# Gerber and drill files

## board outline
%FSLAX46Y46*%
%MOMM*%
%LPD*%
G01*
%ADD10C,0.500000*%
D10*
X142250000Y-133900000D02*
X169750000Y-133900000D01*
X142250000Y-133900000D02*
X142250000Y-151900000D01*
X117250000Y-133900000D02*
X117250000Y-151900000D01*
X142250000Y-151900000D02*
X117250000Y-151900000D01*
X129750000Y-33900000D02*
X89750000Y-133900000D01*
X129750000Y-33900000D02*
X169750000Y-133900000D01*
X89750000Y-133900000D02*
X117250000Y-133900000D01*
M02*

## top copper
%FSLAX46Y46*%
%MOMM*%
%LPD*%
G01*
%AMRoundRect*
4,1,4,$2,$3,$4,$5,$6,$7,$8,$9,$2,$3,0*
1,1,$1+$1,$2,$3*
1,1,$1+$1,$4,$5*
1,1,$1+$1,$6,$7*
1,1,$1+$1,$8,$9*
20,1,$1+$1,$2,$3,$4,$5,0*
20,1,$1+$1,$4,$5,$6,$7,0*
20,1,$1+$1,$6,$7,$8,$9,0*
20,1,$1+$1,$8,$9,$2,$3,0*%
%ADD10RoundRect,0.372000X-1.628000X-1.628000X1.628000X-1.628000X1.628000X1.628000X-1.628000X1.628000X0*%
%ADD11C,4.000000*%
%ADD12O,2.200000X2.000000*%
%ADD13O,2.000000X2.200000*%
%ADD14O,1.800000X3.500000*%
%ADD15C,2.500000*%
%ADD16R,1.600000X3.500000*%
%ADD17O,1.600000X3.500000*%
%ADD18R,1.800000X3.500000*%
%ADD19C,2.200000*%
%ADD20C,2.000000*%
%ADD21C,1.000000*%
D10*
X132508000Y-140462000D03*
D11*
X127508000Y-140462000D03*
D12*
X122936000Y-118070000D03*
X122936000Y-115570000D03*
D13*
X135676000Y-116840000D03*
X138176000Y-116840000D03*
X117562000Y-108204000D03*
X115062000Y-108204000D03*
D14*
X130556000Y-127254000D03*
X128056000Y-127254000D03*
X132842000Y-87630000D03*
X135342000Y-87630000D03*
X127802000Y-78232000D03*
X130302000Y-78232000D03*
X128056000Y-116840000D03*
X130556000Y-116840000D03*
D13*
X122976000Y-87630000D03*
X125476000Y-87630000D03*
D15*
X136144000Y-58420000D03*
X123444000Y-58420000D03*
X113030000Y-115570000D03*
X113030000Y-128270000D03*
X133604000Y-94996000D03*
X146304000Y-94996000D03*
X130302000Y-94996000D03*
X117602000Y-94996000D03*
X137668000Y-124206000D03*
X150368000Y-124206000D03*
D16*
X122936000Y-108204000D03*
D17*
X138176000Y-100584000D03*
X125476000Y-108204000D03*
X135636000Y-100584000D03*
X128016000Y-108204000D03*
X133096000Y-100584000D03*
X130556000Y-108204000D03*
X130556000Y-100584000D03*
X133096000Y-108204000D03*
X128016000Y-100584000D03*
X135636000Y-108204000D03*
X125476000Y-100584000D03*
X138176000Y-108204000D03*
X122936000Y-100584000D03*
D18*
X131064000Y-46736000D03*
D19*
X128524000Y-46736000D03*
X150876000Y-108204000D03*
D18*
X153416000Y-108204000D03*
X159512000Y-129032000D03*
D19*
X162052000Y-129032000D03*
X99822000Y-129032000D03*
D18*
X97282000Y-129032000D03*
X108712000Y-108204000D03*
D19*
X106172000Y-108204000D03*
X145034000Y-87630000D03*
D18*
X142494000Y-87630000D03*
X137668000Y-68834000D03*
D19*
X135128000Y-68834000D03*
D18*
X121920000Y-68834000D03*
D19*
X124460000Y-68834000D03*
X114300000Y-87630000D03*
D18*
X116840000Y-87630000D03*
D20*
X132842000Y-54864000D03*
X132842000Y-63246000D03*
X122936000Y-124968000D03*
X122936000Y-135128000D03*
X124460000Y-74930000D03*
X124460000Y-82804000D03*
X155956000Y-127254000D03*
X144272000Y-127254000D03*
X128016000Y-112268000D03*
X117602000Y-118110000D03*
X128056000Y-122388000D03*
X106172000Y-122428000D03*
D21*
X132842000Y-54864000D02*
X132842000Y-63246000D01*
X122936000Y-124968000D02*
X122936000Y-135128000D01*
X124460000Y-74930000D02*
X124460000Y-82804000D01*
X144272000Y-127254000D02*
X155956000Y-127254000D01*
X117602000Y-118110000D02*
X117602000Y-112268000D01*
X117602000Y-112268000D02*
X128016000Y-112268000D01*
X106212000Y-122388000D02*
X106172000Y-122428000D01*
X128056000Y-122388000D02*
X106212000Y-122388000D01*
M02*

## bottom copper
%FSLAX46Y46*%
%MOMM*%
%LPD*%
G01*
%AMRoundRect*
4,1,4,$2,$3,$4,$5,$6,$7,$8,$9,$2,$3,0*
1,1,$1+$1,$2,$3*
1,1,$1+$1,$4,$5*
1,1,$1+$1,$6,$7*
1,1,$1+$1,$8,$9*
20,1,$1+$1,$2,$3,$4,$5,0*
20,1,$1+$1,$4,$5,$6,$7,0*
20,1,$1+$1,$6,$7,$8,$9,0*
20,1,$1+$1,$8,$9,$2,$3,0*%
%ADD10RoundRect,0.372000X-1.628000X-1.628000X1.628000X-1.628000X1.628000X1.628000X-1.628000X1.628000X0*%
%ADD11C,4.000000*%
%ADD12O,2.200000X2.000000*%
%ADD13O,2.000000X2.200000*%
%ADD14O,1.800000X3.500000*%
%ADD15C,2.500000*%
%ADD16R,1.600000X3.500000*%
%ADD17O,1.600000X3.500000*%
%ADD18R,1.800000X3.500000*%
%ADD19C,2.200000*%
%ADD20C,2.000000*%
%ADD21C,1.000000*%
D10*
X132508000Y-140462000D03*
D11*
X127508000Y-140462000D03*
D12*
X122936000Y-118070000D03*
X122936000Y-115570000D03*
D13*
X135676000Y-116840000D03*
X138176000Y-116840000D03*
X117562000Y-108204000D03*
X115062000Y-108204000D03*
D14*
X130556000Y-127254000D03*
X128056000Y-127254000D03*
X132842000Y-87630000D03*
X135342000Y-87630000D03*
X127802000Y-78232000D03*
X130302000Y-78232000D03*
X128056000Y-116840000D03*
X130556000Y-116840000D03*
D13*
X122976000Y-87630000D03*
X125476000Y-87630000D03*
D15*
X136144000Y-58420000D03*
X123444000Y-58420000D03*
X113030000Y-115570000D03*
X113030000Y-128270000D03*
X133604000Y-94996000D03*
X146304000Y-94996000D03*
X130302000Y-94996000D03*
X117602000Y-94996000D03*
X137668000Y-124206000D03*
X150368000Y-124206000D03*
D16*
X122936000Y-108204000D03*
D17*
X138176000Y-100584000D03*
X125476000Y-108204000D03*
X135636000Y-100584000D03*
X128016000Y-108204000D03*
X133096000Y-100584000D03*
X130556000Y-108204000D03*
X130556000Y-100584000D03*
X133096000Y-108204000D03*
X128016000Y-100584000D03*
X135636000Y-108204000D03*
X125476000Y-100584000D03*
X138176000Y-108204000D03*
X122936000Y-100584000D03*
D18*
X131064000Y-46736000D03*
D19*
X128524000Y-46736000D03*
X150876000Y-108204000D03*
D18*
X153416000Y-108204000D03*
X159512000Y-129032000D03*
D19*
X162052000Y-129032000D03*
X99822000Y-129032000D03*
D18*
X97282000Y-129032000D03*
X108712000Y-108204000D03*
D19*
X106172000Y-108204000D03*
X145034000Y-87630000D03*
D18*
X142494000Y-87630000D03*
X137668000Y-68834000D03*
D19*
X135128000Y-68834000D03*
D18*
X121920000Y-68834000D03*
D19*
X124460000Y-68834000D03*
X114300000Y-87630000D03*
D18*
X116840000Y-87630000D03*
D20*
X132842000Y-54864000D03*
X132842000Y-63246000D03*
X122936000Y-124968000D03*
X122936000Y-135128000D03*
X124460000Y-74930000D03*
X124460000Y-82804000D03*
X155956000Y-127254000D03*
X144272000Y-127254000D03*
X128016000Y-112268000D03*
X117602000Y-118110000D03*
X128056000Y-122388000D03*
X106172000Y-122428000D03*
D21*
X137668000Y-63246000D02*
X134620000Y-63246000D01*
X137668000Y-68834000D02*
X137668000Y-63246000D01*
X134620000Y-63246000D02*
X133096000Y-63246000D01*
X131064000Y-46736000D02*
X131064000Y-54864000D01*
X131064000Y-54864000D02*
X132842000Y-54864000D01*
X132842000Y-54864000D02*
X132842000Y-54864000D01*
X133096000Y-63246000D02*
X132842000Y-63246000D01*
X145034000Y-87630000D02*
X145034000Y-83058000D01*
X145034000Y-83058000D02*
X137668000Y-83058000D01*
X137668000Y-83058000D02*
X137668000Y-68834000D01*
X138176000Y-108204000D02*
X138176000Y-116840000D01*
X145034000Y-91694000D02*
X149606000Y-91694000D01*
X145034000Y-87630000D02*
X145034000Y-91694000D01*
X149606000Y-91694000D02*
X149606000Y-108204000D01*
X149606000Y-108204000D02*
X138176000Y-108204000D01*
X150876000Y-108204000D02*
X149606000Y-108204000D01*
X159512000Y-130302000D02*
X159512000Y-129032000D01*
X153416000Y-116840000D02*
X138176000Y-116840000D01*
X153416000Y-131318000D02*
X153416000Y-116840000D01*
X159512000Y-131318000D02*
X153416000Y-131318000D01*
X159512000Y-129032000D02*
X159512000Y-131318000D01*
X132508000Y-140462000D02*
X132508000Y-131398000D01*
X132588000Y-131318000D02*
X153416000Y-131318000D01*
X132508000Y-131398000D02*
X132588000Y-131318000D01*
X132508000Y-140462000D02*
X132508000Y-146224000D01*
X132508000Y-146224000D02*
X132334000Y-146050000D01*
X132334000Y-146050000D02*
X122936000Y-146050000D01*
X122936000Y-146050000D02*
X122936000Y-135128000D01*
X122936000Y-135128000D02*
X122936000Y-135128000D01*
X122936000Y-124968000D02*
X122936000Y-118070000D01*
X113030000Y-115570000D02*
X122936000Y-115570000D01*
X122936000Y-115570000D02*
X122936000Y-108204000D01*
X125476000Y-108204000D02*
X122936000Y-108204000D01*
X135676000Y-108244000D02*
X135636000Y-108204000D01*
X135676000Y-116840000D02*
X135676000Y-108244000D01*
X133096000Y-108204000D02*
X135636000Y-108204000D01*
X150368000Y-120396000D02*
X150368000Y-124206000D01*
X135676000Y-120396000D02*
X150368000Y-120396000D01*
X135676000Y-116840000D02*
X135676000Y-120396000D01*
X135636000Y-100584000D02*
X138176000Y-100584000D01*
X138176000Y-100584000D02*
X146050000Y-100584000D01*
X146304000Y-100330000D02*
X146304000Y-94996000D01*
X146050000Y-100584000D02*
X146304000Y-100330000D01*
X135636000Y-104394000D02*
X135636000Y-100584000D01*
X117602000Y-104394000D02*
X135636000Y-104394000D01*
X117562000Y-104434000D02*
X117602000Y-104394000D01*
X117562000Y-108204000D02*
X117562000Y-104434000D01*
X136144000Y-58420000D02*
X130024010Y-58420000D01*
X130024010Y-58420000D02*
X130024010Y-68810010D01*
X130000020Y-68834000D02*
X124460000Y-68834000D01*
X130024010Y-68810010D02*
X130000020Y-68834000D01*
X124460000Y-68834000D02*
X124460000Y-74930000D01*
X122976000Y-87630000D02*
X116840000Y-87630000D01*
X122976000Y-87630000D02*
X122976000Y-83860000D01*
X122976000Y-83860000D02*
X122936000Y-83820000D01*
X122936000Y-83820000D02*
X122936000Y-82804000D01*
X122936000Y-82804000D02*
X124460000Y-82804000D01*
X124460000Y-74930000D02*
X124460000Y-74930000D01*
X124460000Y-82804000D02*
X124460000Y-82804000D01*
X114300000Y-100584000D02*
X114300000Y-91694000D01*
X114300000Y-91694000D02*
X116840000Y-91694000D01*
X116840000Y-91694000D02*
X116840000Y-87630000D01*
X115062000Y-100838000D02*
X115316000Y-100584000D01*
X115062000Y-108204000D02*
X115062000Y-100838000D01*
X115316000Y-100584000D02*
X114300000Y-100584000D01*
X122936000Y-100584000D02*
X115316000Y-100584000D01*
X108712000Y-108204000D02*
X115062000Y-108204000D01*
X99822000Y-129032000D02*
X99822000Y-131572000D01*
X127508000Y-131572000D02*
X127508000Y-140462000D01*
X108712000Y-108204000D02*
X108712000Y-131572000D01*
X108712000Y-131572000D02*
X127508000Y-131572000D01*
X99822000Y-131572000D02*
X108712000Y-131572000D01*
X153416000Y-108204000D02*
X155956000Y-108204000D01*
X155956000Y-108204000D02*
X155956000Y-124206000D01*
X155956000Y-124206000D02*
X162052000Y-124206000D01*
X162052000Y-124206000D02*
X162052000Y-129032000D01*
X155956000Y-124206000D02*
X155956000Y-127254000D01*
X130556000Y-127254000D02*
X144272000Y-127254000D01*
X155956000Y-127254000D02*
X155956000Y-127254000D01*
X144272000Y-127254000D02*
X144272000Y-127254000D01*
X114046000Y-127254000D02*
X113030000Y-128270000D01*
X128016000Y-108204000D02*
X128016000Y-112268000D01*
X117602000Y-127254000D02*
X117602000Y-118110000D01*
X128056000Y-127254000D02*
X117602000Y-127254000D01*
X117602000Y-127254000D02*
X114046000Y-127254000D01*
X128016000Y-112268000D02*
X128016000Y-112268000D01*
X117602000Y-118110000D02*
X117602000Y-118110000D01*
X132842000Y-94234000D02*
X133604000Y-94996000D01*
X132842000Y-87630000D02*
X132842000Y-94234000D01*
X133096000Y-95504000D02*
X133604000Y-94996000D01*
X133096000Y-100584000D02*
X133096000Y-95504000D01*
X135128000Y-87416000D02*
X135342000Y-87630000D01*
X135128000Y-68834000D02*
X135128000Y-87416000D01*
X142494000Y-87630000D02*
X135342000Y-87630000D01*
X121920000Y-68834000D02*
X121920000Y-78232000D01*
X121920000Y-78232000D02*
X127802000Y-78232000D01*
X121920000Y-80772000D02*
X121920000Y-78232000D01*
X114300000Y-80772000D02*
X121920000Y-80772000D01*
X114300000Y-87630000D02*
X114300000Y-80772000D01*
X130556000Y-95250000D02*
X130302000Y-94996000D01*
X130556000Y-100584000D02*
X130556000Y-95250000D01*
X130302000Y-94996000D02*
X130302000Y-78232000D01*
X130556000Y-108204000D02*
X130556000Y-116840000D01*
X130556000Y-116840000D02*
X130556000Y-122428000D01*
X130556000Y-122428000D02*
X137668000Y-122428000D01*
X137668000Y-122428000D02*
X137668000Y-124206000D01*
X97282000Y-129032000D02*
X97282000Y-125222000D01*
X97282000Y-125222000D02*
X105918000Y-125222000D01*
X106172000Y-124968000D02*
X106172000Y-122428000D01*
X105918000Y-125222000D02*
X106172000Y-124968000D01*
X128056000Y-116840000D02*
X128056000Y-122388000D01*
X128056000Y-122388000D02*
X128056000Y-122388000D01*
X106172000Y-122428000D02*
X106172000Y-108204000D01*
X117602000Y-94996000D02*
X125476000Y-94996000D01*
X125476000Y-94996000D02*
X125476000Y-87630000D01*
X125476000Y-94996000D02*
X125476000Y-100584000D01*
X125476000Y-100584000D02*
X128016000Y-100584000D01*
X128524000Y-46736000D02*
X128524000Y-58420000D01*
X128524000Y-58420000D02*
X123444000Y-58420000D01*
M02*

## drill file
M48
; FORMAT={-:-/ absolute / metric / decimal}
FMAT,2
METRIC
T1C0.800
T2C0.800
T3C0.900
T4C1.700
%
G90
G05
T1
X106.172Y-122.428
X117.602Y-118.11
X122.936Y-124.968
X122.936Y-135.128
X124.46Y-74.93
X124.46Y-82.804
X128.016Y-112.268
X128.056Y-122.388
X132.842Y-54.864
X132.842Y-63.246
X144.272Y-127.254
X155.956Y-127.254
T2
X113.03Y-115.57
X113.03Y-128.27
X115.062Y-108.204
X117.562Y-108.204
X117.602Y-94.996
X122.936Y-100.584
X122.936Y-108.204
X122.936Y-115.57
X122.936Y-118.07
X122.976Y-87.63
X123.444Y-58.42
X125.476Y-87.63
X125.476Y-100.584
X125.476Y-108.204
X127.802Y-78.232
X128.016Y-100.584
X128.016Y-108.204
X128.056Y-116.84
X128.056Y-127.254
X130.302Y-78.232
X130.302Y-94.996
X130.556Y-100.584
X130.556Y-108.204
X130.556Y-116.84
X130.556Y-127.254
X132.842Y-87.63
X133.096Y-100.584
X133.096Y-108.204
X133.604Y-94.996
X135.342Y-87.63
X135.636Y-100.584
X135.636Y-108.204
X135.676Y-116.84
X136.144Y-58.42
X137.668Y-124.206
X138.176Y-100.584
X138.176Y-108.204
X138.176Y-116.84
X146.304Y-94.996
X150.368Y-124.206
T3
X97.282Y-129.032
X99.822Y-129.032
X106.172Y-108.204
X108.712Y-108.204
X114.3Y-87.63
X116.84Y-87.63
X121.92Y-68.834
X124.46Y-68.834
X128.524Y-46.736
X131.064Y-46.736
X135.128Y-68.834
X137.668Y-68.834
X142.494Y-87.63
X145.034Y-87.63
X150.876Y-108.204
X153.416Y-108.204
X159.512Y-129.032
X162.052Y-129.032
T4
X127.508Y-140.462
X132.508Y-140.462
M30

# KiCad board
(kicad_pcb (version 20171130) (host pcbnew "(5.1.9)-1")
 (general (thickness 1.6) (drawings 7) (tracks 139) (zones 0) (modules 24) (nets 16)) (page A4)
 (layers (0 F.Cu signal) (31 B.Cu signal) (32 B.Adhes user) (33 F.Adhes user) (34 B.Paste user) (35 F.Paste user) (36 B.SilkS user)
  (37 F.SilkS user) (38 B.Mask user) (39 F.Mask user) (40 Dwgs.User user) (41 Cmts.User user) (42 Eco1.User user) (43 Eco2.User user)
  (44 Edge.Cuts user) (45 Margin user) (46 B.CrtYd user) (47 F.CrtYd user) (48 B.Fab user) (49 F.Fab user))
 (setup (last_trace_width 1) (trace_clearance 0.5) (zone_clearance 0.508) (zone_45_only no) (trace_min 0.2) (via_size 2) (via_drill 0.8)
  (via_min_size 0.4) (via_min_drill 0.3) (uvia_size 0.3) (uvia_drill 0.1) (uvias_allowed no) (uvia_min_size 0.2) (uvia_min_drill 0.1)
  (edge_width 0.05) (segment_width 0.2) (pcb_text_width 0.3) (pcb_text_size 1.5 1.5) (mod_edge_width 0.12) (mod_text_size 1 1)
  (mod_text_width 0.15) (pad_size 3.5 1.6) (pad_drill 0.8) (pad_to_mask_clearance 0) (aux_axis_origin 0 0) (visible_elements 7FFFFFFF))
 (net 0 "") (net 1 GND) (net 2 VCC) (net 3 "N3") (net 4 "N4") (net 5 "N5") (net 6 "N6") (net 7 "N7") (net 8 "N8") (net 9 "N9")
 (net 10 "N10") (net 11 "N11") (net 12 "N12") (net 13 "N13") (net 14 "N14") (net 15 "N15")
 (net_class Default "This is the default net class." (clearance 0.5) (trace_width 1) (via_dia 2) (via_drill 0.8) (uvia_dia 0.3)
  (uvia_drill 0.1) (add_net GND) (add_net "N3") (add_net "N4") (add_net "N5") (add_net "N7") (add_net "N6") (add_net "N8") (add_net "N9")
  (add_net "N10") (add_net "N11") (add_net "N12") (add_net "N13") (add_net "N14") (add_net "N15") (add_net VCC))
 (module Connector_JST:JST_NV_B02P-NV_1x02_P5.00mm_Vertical (layer F.Cu) (at 127.508 140.462)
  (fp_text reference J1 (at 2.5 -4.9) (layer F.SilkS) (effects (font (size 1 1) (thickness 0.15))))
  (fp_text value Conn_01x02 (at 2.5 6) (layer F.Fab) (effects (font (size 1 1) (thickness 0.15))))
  (pad 2 thru_hole roundrect (at 5 0) (size 4 4) (drill 1.7) (layers *.Cu *.Mask) (roundrect_rratio 0.09300000000000001) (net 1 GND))
  (pad 1 thru_hole circle (at 0 0) (size 4 4) (drill 1.7) (layers *.Cu *.Mask) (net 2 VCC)))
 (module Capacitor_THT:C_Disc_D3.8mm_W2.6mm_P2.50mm (layer F.Cu) (at 122.936 115.57 270)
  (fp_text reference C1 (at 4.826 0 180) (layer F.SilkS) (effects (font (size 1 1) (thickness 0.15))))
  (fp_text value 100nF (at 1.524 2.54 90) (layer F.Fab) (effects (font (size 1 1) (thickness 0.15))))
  (pad 2 thru_hole oval (at 2.5 0 270) (size 2 2.2) (drill 0.8) (layers *.Cu *.Mask) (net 1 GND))
  (pad 1 thru_hole oval (at 0 0 270) (size 2 2.2) (drill 0.8) (layers *.Cu *.Mask) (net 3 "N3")))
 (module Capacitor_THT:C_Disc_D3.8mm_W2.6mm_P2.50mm (layer F.Cu) (at 135.676 116.84)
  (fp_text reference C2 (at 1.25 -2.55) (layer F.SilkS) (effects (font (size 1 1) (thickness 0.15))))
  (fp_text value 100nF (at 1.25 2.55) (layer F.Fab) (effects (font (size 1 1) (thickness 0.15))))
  (pad 1 thru_hole oval (at 0 0) (size 2 2.2) (drill 0.8) (layers *.Cu *.Mask) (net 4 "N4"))
  (pad 2 thru_hole oval (at 2.5 0) (size 2 2.2) (drill 0.8) (layers *.Cu *.Mask) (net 1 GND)))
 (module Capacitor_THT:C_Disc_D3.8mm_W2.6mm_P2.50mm (layer F.Cu) (at 115.062 108.204)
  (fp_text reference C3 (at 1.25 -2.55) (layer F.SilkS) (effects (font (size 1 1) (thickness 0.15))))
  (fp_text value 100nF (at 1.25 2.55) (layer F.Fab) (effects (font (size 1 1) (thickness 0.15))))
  (pad 2 thru_hole oval (at 2.5 0) (size 2 2.2) (drill 0.8) (layers *.Cu *.Mask) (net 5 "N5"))
  (pad 1 thru_hole oval (at 0 0) (size 2 2.2) (drill 0.8) (layers *.Cu *.Mask) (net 2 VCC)))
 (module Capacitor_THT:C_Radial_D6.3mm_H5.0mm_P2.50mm (layer F.Cu) (at 128.056 127.254)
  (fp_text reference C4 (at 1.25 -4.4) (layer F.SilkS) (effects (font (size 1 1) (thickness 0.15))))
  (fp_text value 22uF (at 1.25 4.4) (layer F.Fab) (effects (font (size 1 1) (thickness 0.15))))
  (pad 2 thru_hole oval (at 2.5 0) (size 1.8 3.5) (drill 0.8) (layers *.Cu *.Mask) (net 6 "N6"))
  (pad 1 thru_hole oval (at 0 0) (size 1.8 3.5) (drill 0.8) (layers *.Cu *.Mask) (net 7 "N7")))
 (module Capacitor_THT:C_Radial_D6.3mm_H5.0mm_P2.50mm (layer F.Cu) (at 132.842 87.63)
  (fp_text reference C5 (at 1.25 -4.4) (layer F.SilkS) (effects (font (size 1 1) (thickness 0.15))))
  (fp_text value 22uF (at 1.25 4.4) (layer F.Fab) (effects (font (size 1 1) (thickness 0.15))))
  (pad 1 thru_hole oval (at 0 0) (size 1.8 3.5) (drill 0.8) (layers *.Cu *.Mask) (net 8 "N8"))
  (pad 2 thru_hole oval (at 2.5 0) (size 1.8 3.5) (drill 0.8) (layers *.Cu *.Mask) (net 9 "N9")))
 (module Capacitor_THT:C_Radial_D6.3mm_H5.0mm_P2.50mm (layer F.Cu) (at 127.802 78.232)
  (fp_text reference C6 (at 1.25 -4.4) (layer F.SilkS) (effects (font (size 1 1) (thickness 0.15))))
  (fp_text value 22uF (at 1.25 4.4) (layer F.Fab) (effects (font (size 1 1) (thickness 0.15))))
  (pad 1 thru_hole oval (at 0 0) (size 1.8 3.5) (drill 0.8) (layers *.Cu *.Mask) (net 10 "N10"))
  (pad 2 thru_hole oval (at 2.5 0) (size 1.8 3.5) (drill 0.8) (layers *.Cu *.Mask) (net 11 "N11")))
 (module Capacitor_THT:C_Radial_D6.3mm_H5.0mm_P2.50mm (layer F.Cu) (at 128.056 116.84)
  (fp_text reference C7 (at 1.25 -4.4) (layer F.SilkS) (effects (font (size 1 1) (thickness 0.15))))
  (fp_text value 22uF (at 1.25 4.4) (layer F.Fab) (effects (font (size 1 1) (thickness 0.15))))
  (pad 1 thru_hole oval (at 0 0) (size 1.8 3.5) (drill 0.8) (layers *.Cu *.Mask) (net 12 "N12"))
  (pad 2 thru_hole oval (at 2.5 0) (size 1.8 3.5) (drill 0.8) (layers *.Cu *.Mask) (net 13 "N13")))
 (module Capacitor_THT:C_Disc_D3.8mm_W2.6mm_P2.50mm (layer F.Cu) (at 122.976 87.63)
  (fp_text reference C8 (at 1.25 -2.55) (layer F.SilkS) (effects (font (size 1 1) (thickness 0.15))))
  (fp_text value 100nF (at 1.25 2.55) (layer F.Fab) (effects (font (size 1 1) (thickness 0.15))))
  (pad 1 thru_hole oval (at 0 0) (size 2 2.2) (drill 0.8) (layers *.Cu *.Mask) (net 2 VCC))
  (pad 2 thru_hole oval (at 2.5 0) (size 2 2.2) (drill 0.8) (layers *.Cu *.Mask) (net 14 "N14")))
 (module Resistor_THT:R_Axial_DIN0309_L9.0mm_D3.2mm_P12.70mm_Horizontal (layer F.Cu) (at 136.144 58.42 180)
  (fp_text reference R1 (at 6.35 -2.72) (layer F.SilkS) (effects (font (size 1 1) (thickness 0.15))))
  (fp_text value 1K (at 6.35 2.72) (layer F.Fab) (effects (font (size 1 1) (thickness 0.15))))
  (pad 1 thru_hole circle (at 0 0 180) (size 2.5 2.5) (drill 0.8) (layers *.Cu *.Mask) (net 2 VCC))
  (pad 2 thru_hole circle (at 12.7 0 180) (size 2.5 2.5) (drill 0.8) (layers *.Cu *.Mask) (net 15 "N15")))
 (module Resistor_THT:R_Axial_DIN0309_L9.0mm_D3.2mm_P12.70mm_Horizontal (layer F.Cu) (at 113.03 128.27 90)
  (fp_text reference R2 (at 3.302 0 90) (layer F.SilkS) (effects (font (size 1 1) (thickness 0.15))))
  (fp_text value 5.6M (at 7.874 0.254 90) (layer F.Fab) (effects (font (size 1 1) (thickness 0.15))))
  (pad 2 thru_hole circle (at 12.7 0 90) (size 2.5 2.5) (drill 0.8) (layers *.Cu *.Mask) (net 3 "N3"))
  (pad 1 thru_hole circle (at 0 0 90) (size 2.5 2.5) (drill 0.8) (layers *.Cu *.Mask) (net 7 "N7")))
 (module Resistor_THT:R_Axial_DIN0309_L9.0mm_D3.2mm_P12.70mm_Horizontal (layer F.Cu) (at 133.604 94.996)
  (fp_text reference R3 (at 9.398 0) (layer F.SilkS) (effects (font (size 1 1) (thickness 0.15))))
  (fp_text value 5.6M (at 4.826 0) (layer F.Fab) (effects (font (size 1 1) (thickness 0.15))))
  (pad 1 thru_hole circle (at 0 0) (size 2.5 2.5) (drill 0.8) (layers *.Cu *.Mask) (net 8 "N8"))
  (pad 2 thru_hole circle (at 12.7 0) (size 2.5 2.5) (drill 0.8) (layers *.Cu *.Mask) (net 5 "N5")))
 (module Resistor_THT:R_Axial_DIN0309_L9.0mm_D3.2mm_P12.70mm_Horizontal (layer F.Cu) (at 130.302 94.996 180)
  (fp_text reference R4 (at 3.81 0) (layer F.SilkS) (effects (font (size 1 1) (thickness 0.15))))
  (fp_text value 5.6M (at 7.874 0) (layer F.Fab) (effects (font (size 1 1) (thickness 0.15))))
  (pad 1 thru_hole circle (at 0 0 180) (size 2.5 2.5) (drill 0.8) (layers *.Cu *.Mask) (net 11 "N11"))
  (pad 2 thru_hole circle (at 12.7 0 180) (size 2.5 2.5) (drill 0.8) (layers *.Cu *.Mask) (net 14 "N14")))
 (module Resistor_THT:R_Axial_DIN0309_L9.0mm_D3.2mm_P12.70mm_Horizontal (layer F.Cu) (at 137.668 124.206)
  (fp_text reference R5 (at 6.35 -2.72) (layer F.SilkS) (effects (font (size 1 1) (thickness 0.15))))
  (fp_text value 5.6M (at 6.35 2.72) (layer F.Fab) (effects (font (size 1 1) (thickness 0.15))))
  (pad 1 thru_hole circle (at 0 0) (size 2.5 2.5) (drill 0.8) (layers *.Cu *.Mask) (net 13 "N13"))
  (pad 2 thru_hole circle (at 12.7 0) (size 2.5 2.5) (drill 0.8) (layers *.Cu *.Mask) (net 4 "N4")))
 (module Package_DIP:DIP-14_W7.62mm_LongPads (layer F.Cu) (at 122.936 108.204 90)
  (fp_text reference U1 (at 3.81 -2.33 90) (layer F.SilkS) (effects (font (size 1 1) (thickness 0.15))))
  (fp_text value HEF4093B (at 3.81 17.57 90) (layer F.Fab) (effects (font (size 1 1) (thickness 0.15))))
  (pad 1 thru_hole rect (at 0 0 90) (size 3.5 1.6) (drill 0.8) (layers *.Cu *.Mask) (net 3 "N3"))
  (pad 8 thru_hole oval (at 7.62 15.24 90) (size 3.5 1.6) (drill 0.8) (layers *.Cu *.Mask) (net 5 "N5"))
  (pad 2 thru_hole oval (at 0 2.54 90) (size 3.5 1.6) (drill 0.8) (layers *.Cu *.Mask) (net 3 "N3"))
  (pad 9 thru_hole oval (at 7.62 12.7 90) (size 3.5 1.6) (drill 0.8) (layers *.Cu *.Mask) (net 5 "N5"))
  (pad 3 thru_hole oval (at 0 5.08 90) (size 3.5 1.6) (drill 0.8) (layers *.Cu *.Mask) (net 7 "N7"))
  (pad 10 thru_hole oval (at 7.62 10.16 90) (size 3.5 1.6) (drill 0.8) (layers *.Cu *.Mask) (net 8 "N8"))
  (pad 4 thru_hole oval (at 0 7.62 90) (size 3.5 1.6) (drill 0.8) (layers *.Cu *.Mask) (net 13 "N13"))
  (pad 11 thru_hole oval (at 7.62 7.62 90) (size 3.5 1.6) (drill 0.8) (layers *.Cu *.Mask) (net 11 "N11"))
  (pad 5 thru_hole oval (at 0 10.16 90) (size 3.5 1.6) (drill 0.8) (layers *.Cu *.Mask) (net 4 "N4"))
  (pad 12 thru_hole oval (at 7.62 5.08 90) (size 3.5 1.6) (drill 0.8) (layers *.Cu *.Mask) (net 14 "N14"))
  (pad 6 thru_hole oval (at 0 12.7 90) (size 3.5 1.6) (drill 0.8) (layers *.Cu *.Mask) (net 4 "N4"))
  (pad 13 thru_hole oval (at 7.62 2.54 90) (size 3.5 1.6) (drill 0.8) (layers *.Cu *.Mask) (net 14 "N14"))
  (pad 7 thru_hole oval (at 0 15.24 90) (size 3.5 1.6) (drill 0.8) (layers *.Cu *.Mask) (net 1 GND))
  (pad 14 thru_hole oval (at 7.62 0 90) (size 3.5 1.6) (drill 0.8) (layers *.Cu *.Mask) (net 2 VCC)))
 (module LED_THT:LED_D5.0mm (layer F.Cu) (at 131.064 46.736 180)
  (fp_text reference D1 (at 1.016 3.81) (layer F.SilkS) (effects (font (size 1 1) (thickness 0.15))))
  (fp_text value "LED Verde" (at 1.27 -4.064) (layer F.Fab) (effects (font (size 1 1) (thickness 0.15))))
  (pad 1 thru_hole rect (at 0 0 180) (size 1.8 3.5) (drill 0.9) (layers *.Cu *.Mask) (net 1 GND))
  (pad 2 thru_hole circle (at 2.54 0 180) (size 2.2 2.2) (drill 0.9) (layers *.Cu *.Mask) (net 15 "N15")))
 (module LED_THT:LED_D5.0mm (layer F.Cu) (at 153.416 108.204 180)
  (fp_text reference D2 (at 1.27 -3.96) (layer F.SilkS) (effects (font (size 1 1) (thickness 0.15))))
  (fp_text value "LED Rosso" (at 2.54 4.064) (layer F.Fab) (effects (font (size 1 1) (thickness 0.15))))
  (pad 2 thru_hole circle (at 2.54 0 180) (size 2.2 2.2) (drill 0.9) (layers *.Cu *.Mask) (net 1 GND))
  (pad 1 thru_hole rect (at 0 0 180) (size 1.8 3.5) (drill 0.9) (layers *.Cu *.Mask) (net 6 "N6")))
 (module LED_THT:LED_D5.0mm (layer F.Cu) (at 159.512 129.032)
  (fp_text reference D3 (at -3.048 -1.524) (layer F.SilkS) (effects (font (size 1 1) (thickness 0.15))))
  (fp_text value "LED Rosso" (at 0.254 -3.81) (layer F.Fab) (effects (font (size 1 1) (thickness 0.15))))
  (pad 1 thru_hole rect (at 0 0) (size 1.8 3.5) (drill 0.9) (layers *.Cu *.Mask) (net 1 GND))
  (pad 2 thru_hole circle (at 2.54 0) (size 2.2 2.2) (drill 0.9) (layers *.Cu *.Mask) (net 6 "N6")))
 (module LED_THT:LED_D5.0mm (layer F.Cu) (at 97.282 129.032)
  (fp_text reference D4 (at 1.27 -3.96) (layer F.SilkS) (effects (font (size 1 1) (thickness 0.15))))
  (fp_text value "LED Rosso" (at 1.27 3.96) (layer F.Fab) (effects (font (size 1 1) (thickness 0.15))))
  (pad 2 thru_hole circle (at 2.54 0) (size 2.2 2.2) (drill 0.9) (layers *.Cu *.Mask) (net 2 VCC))
  (pad 1 thru_hole rect (at 0 0) (size 1.8 3.5) (drill 0.9) (layers *.Cu *.Mask) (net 12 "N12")))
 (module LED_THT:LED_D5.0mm (layer F.Cu) (at 108.712 108.204 180)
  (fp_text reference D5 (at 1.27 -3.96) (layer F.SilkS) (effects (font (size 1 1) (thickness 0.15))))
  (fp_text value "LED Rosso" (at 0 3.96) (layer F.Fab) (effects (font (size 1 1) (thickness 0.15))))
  (pad 1 thru_hole rect (at 0 0 180) (size 1.8 3.5) (drill 0.9) (layers *.Cu *.Mask) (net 2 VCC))
  (pad 2 thru_hole circle (at 2.54 0 180) (size 2.2 2.2) (drill 0.9) (layers *.Cu *.Mask) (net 12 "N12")))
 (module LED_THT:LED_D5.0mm (layer F.Cu) (at 142.494 87.63)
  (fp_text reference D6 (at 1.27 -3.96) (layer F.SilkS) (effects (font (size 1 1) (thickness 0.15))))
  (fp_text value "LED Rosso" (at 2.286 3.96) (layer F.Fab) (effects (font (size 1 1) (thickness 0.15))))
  (pad 2 thru_hole circle (at 2.54 0) (size 2.2 2.2) (drill 0.9) (layers *.Cu *.Mask) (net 1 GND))
  (pad 1 thru_hole rect (at 0 0) (size 1.8 3.5) (drill 0.9) (layers *.Cu *.Mask) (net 9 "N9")))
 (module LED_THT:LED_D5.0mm (layer F.Cu) (at 137.668 68.834 180)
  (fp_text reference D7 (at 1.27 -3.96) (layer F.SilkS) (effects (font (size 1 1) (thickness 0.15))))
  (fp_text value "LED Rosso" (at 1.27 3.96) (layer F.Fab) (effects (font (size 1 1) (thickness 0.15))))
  (pad 1 thru_hole rect (at 0 0 180) (size 1.8 3.5) (drill 0.9) (layers *.Cu *.Mask) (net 1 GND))
  (pad 2 thru_hole circle (at 2.54 0 180) (size 2.2 2.2) (drill 0.9) (layers *.Cu *.Mask) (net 9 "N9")))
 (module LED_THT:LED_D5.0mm (layer F.Cu) (at 121.92 68.834)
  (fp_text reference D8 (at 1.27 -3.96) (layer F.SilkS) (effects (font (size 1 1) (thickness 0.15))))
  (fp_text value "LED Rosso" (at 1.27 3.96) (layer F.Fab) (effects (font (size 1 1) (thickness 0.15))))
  (pad 1 thru_hole rect (at 0 0) (size 1.8 3.5) (drill 0.9) (layers *.Cu *.Mask) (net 10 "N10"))
  (pad 2 thru_hole circle (at 2.54 0) (size 2.2 2.2) (drill 0.9) (layers *.Cu *.Mask) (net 2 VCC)))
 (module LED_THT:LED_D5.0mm (layer F.Cu) (at 116.84 87.63 180)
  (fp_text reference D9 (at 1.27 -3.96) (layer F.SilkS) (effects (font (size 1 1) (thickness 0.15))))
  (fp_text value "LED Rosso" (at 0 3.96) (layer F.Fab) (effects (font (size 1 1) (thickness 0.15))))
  (pad 2 thru_hole circle (at 2.54 0 180) (size 2.2 2.2) (drill 0.9) (layers *.Cu *.Mask) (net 10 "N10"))
  (pad 1 thru_hole rect (at 0 0 180) (size 1.8 3.5) (drill 0.9) (layers *.Cu *.Mask) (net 2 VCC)))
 (gr_line (start 142.25 133.9) (end 169.75 133.9) (layer Edge.Cuts) (width 0.5))
 (gr_line (start 142.25 133.9) (end 142.25 151.9) (layer Edge.Cuts) (width 0.5))
 (gr_line (start 117.25 133.9) (end 117.25 151.9) (layer Edge.Cuts) (width 0.5))
 (gr_line (start 142.25 151.9) (end 117.25 151.9) (layer Edge.Cuts) (width 0.5))
 (gr_line (start 129.75 33.9) (end 89.75 133.9) (layer Edge.Cuts) (width 0.5))
 (gr_line (start 129.75 33.9) (end 169.75 133.9) (layer Edge.Cuts) (width 0.5))
 (gr_line (start 89.75 133.9) (end 117.25 133.9) (layer Edge.Cuts) (width 0.5))
 (segment (start 137.668 63.246) (end 134.62 63.246) (width 1) (layer B.Cu) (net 1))
 (segment (start 137.668 68.834) (end 137.668 63.246) (width 1) (layer B.Cu) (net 1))
 (segment (start 134.62 63.246) (end 133.096 63.246) (width 1) (layer B.Cu) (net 1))
 (segment (start 131.064 46.736) (end 131.064 54.864) (width 1) (layer B.Cu) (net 1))
 (segment (start 131.064 54.864) (end 132.842 54.864) (width 1) (layer B.Cu) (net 1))
 (segment (start 132.842 54.864) (end 132.842 54.864) (width 1) (layer B.Cu) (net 1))
 (via (at 132.842 54.864) (size 2) (drill 0.8) (layers F.Cu B.Cu) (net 1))
 (segment (start 133.096 63.246) (end 132.842 63.246) (width 1) (layer B.Cu) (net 1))
 (via (at 132.842 63.246) (size 2) (drill 0.8) (layers F.Cu B.Cu) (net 1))
 (segment (start 132.842 54.864) (end 132.842 63.246) (width 1) (layer F.Cu) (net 1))
 (segment (start 145.034 87.63) (end 145.034 83.058) (width 1) (layer B.Cu) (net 1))
 (segment (start 145.034 83.058) (end 137.668 83.058) (width 1) (layer B.Cu) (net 1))
 (segment (start 137.668 83.058) (end 137.668 68.834) (width 1) (layer B.Cu) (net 1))
 (segment (start 138.176 108.204) (end 138.176 116.84) (width 1) (layer B.Cu) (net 1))
 (segment (start 145.034 91.694) (end 149.606 91.694) (width 1) (layer B.Cu) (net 1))
 (segment (start 145.034 87.63) (end 145.034 91.694) (width 1) (layer B.Cu) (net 1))
 (segment (start 149.606 91.694) (end 149.606 108.204) (width 1) (layer B.Cu) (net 1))
 (segment (start 149.606 108.204) (end 138.176 108.204) (width 1) (layer B.Cu) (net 1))
 (segment (start 150.876 108.204) (end 149.606 108.204) (width 1) (layer B.Cu) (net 1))
 (segment (start 159.512 130.302) (end 159.512 129.032) (width 1) (layer B.Cu) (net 1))
 (segment (start 153.416 116.84) (end 138.176 116.84) (width 1) (layer B.Cu) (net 1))
 (segment (start 153.416 131.318) (end 153.416 116.84) (width 1) (layer B.Cu) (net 1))
 (segment (start 159.512 131.318) (end 153.416 131.318) (width 1) (layer B.Cu) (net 1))
 (segment (start 159.512 129.032) (end 159.512 131.318) (width 1) (layer B.Cu) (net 1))
 (segment (start 132.508 140.462) (end 132.508 131.398) (width 1) (layer B.Cu) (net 1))
 (segment (start 132.588 131.318) (end 153.416 131.318) (width 1) (layer B.Cu) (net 1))
 (segment (start 132.508 131.398) (end 132.588 131.318) (width 1) (layer B.Cu) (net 1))
 (segment (start 132.508 140.462) (end 132.508 146.224) (width 1) (layer B.Cu) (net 1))
 (segment (start 132.508 146.224) (end 132.334 146.05) (width 1) (layer B.Cu) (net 1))
 (segment (start 132.334 146.05) (end 122.936 146.05) (width 1) (layer B.Cu) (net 1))
 (segment (start 122.936 146.05) (end 122.936 135.128) (width 1) (layer B.Cu) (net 1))
 (via (at 122.936 124.968) (size 2) (drill 0.8) (layers F.Cu B.Cu) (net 1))
 (segment (start 122.936 135.128) (end 122.936 135.128) (width 1) (layer B.Cu) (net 1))
 (via (at 122.936 135.128) (size 2) (drill 0.8) (layers F.Cu B.Cu) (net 1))
 (segment (start 122.936 124.968) (end 122.936 118.07) (width 1) (layer B.Cu) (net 1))
 (segment (start 122.936 124.968) (end 122.936 135.128) (width 1) (layer F.Cu) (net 1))
 (segment (start 113.03 115.57) (end 122.936 115.57) (width 1) (layer B.Cu) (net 3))
 (segment (start 122.936 115.57) (end 122.936 108.204) (width 1) (layer B.Cu) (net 3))
 (segment (start 125.476 108.204) (end 122.936 108.204) (width 1) (layer B.Cu) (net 3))
 (segment (start 135.676 108.244) (end 135.636 108.204) (width 1) (layer B.Cu) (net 4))
 (segment (start 135.676 116.84) (end 135.676 108.244) (width 1) (layer B.Cu) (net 4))
 (segment (start 133.096 108.204) (end 135.636 108.204) (width 1) (layer B.Cu) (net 4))
 (segment (start 150.368 120.396) (end 150.368 124.206) (width 1) (layer B.Cu) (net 4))
 (segment (start 135.676 120.396) (end 150.368 120.396) (width 1) (layer B.Cu) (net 4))
 (segment (start 135.676 116.84) (end 135.676 120.396) (width 1) (layer B.Cu) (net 4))
 (segment (start 135.636 100.584) (end 138.176 100.584) (width 1) (layer B.Cu) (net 5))
 (segment (start 138.176 100.584) (end 146.05 100.584) (width 1) (layer B.Cu) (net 5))
 (segment (start 146.304 100.33) (end 146.304 94.996) (width 1) (layer B.Cu) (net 5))
 (segment (start 146.05 100.584) (end 146.304 100.33) (width 1) (layer B.Cu) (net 5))
 (segment (start 135.636 104.394) (end 135.636 100.584) (width 1) (layer B.Cu) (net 5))
 (segment (start 117.602 104.394) (end 135.636 104.394) (width 1) (layer B.Cu) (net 5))
 (segment (start 117.562 104.434) (end 117.602 104.394) (width 1) (layer B.Cu) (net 5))
 (segment (start 117.562 108.204) (end 117.562 104.434) (width 1) (layer B.Cu) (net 5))
 (segment (start 136.144 58.42) (end 130.02401 58.42) (width 1) (layer B.Cu) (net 2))
 (segment (start 130.02401 58.42) (end 130.02401 68.81001) (width 1) (layer B.Cu) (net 2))
 (segment (start 130.00002 68.834) (end 124.46 68.834) (width 1) (layer B.Cu) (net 2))
 (segment (start 130.02401 68.81001) (end 130.00002 68.834) (width 1) (layer B.Cu) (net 2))
 (segment (start 124.46 68.834) (end 124.46 74.93) (width 1) (layer B.Cu) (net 2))
 (segment (start 122.976 87.63) (end 116.84 87.63) (width 1) (layer B.Cu) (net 2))
 (segment (start 122.976 87.63) (end 122.976 83.86) (width 1) (layer B.Cu) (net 2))
 (segment (start 122.976 83.86) (end 122.936 83.82) (width 1) (layer B.Cu) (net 2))
 (segment (start 122.936 83.82) (end 122.936 82.804) (width 1) (layer B.Cu) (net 2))
 (segment (start 122.936 82.804) (end 124.46 82.804) (width 1) (layer B.Cu) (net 2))
 (segment (start 124.46 74.93) (end 124.46 74.93) (width 1) (layer B.Cu) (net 2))
 (via (at 124.46 74.93) (size 2) (drill 0.8) (layers F.Cu B.Cu) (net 2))
 (segment (start 124.46 82.804) (end 124.46 82.804) (width 1) (layer B.Cu) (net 2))
 (via (at 124.46 82.804) (size 2) (drill 0.8) (layers F.Cu B.Cu) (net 2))
 (segment (start 124.46 74.93) (end 124.46 82.804) (width 1) (layer F.Cu) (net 2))
 (segment (start 114.3 100.584) (end 114.3 91.694) (width 1) (layer B.Cu) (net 2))
 (segment (start 114.3 91.694) (end 116.84 91.694) (width 1) (layer B.Cu) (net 2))
 (segment (start 116.84 91.694) (end 116.84 87.63) (width 1) (layer B.Cu) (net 2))
 (segment (start 115.062 100.838) (end 115.316 100.584) (width 1) (layer B.Cu) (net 2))
 (segment (start 115.062 108.204) (end 115.062 100.838) (width 1) (layer B.Cu) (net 2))
 (segment (start 115.316 100.584) (end 114.3 100.584) (width 1) (layer B.Cu) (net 2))
 (segment (start 122.936 100.584) (end 115.316 100.584) (width 1) (layer B.Cu) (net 2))
 (segment (start 108.712 108.204) (end 115.062 108.204) (width 1) (layer B.Cu) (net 2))
 (segment (start 99.822 129.032) (end 99.822 131.572) (width 1) (layer B.Cu) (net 2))
 (segment (start 127.508 131.572) (end 127.508 140.462) (width 1) (layer B.Cu) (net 2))
 (segment (start 108.712 108.204) (end 108.712 131.572) (width 1) (layer B.Cu) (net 2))
 (segment (start 108.712 131.572) (end 127.508 131.572) (width 1) (layer B.Cu) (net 2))
 (segment (start 99.822 131.572) (end 108.712 131.572) (width 1) (layer B.Cu) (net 2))
 (segment (start 153.416 108.204) (end 155.956 108.204) (width 1) (layer B.Cu) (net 6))
 (segment (start 155.956 108.204) (end 155.956 124.206) (width 1) (layer B.Cu) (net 6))
 (segment (start 155.956 124.206) (end 162.052 124.206) (width 1) (layer B.Cu) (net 6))
 (segment (start 162.052 124.206) (end 162.052 129.032) (width 1) (layer B.Cu) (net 6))
 (segment (start 155.956 124.206) (end 155.956 127.254) (width 1) (layer B.Cu) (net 6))
 (segment (start 130.556 127.254) (end 144.272 127.254) (width 1) (layer B.Cu) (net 6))
 (segment (start 155.956 127.254) (end 155.956 127.254) (width 1) (layer B.Cu) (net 6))
 (via (at 155.956 127.254) (size 2) (drill 0.8) (layers F.Cu B.Cu) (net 6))
 (segment (start 144.272 127.254) (end 144.272 127.254) (width 1) (layer B.Cu) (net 6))
 (via (at 144.272 127.254) (size 2) (drill 0.8) (layers F.Cu B.Cu) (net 6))
 (segment (start 144.272 127.254) (end 155.956 127.254) (width 1) (layer F.Cu) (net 6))
 (segment (start 114.046 127.254) (end 113.03 128.27) (width 1) (layer B.Cu) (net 7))
 (segment (start 128.016 108.204) (end 128.016 112.268) (width 1) (layer B.Cu) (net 7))
 (segment (start 117.602 127.254) (end 117.602 118.11) (width 1) (layer B.Cu) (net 7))
 (segment (start 128.056 127.254) (end 117.602 127.254) (width 1) (layer B.Cu) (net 7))
 (segment (start 117.602 127.254) (end 114.046 127.254) (width 1) (layer B.Cu) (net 7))
 (segment (start 128.016 112.268) (end 128.016 112.268) (width 1) (layer B.Cu) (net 7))
 (via (at 128.016 112.268) (size 2) (drill 0.8) (layers F.Cu B.Cu) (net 7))
 (segment (start 117.602 118.11) (end 117.602 118.11) (width 1) (layer B.Cu) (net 7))
 (via (at 117.602 118.11) (size 2) (drill 0.8) (layers F.Cu B.Cu) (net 7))
 (segment (start 117.602 118.11) (end 117.602 112.268) (width 1) (layer F.Cu) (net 7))
 (segment (start 117.602 112.268) (end 128.016 112.268) (width 1) (layer F.Cu) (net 7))
 (segment (start 132.842 94.234) (end 133.604 94.996) (width 1) (layer B.Cu) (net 8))
 (segment (start 132.842 87.63) (end 132.842 94.234) (width 1) (layer B.Cu) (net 8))
 (segment (start 133.096 95.504) (end 133.604 94.996) (width 1) (layer B.Cu) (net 8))
 (segment (start 133.096 100.584) (end 133.096 95.504) (width 1) (layer B.Cu) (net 8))
 (segment (start 135.128 87.416) (end 135.342 87.63) (width 1) (layer B.Cu) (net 9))
 (segment (start 135.128 68.834) (end 135.128 87.416) (width 1) (layer B.Cu) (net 9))
 (segment (start 142.494 87.63) (end 135.342 87.63) (width 1) (layer B.Cu) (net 9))
 (segment (start 121.92 68.834) (end 121.92 78.232) (width 1) (layer B.Cu) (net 10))
 (segment (start 121.92 78.232) (end 127.802 78.232) (width 1) (layer B.Cu) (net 10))
 (segment (start 121.92 80.772) (end 121.92 78.232) (width 1) (layer B.Cu) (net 10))
 (segment (start 114.3 80.772) (end 121.92 80.772) (width 1) (layer B.Cu) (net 10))
 (segment (start 114.3 87.63) (end 114.3 80.772) (width 1) (layer B.Cu) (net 10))
 (segment (start 130.556 95.25) (end 130.302 94.996) (width 1) (layer B.Cu) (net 11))
 (segment (start 130.556 100.584) (end 130.556 95.25) (width 1) (layer B.Cu) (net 11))
 (segment (start 130.302 94.996) (end 130.302 78.232) (width 1) (layer B.Cu) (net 11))
 (segment (start 130.556 108.204) (end 130.556 116.84) (width 1) (layer B.Cu) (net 13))
 (segment (start 130.556 116.84) (end 130.556 122.428) (width 1) (layer B.Cu) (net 13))
 (segment (start 130.556 122.428) (end 137.668 122.428) (width 1) (layer B.Cu) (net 13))
 (segment (start 137.668 122.428) (end 137.668 124.206) (width 1) (layer B.Cu) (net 13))
 (segment (start 97.282 129.032) (end 97.282 125.222) (width 1) (layer B.Cu) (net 12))
 (segment (start 97.282 125.222) (end 105.918 125.222) (width 1) (layer B.Cu) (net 12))
 (segment (start 106.172 124.968) (end 106.172 122.428) (width 1) (layer B.Cu) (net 12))
 (segment (start 105.918 125.222) (end 106.172 124.968) (width 1) (layer B.Cu) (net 12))
 (segment (start 128.056 116.84) (end 128.056 122.388) (width 1) (layer B.Cu) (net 12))
 (segment (start 128.056 122.388) (end 128.056 122.388) (width 1) (layer B.Cu) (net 12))
 (via (at 128.056 122.388) (size 2) (drill 0.8) (layers F.Cu B.Cu) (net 12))
 (segment (start 106.172 122.428) (end 106.172 108.204) (width 1) (layer B.Cu) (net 12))
 (via (at 106.172 122.428) (size 2) (drill 0.8) (layers F.Cu B.Cu) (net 12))
 (segment (start 106.212 122.388) (end 106.172 122.428) (width 1) (layer F.Cu) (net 12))
 (segment (start 128.056 122.388) (end 106.212 122.388) (width 1) (layer F.Cu) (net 12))
 (segment (start 117.602 94.996) (end 125.476 94.996) (width 1) (layer B.Cu) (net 14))
 (segment (start 125.476 94.996) (end 125.476 87.63) (width 1) (layer B.Cu) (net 14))
 (segment (start 125.476 94.996) (end 125.476 100.584) (width 1) (layer B.Cu) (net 14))
 (segment (start 125.476 100.584) (end 128.016 100.584) (width 1) (layer B.Cu) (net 14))
 (segment (start 128.524 46.736) (end 128.524 58.42) (width 1) (layer B.Cu) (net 15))
 (segment (start 128.524 58.42) (end 123.444 58.42) (width 1) (layer B.Cu) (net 15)))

